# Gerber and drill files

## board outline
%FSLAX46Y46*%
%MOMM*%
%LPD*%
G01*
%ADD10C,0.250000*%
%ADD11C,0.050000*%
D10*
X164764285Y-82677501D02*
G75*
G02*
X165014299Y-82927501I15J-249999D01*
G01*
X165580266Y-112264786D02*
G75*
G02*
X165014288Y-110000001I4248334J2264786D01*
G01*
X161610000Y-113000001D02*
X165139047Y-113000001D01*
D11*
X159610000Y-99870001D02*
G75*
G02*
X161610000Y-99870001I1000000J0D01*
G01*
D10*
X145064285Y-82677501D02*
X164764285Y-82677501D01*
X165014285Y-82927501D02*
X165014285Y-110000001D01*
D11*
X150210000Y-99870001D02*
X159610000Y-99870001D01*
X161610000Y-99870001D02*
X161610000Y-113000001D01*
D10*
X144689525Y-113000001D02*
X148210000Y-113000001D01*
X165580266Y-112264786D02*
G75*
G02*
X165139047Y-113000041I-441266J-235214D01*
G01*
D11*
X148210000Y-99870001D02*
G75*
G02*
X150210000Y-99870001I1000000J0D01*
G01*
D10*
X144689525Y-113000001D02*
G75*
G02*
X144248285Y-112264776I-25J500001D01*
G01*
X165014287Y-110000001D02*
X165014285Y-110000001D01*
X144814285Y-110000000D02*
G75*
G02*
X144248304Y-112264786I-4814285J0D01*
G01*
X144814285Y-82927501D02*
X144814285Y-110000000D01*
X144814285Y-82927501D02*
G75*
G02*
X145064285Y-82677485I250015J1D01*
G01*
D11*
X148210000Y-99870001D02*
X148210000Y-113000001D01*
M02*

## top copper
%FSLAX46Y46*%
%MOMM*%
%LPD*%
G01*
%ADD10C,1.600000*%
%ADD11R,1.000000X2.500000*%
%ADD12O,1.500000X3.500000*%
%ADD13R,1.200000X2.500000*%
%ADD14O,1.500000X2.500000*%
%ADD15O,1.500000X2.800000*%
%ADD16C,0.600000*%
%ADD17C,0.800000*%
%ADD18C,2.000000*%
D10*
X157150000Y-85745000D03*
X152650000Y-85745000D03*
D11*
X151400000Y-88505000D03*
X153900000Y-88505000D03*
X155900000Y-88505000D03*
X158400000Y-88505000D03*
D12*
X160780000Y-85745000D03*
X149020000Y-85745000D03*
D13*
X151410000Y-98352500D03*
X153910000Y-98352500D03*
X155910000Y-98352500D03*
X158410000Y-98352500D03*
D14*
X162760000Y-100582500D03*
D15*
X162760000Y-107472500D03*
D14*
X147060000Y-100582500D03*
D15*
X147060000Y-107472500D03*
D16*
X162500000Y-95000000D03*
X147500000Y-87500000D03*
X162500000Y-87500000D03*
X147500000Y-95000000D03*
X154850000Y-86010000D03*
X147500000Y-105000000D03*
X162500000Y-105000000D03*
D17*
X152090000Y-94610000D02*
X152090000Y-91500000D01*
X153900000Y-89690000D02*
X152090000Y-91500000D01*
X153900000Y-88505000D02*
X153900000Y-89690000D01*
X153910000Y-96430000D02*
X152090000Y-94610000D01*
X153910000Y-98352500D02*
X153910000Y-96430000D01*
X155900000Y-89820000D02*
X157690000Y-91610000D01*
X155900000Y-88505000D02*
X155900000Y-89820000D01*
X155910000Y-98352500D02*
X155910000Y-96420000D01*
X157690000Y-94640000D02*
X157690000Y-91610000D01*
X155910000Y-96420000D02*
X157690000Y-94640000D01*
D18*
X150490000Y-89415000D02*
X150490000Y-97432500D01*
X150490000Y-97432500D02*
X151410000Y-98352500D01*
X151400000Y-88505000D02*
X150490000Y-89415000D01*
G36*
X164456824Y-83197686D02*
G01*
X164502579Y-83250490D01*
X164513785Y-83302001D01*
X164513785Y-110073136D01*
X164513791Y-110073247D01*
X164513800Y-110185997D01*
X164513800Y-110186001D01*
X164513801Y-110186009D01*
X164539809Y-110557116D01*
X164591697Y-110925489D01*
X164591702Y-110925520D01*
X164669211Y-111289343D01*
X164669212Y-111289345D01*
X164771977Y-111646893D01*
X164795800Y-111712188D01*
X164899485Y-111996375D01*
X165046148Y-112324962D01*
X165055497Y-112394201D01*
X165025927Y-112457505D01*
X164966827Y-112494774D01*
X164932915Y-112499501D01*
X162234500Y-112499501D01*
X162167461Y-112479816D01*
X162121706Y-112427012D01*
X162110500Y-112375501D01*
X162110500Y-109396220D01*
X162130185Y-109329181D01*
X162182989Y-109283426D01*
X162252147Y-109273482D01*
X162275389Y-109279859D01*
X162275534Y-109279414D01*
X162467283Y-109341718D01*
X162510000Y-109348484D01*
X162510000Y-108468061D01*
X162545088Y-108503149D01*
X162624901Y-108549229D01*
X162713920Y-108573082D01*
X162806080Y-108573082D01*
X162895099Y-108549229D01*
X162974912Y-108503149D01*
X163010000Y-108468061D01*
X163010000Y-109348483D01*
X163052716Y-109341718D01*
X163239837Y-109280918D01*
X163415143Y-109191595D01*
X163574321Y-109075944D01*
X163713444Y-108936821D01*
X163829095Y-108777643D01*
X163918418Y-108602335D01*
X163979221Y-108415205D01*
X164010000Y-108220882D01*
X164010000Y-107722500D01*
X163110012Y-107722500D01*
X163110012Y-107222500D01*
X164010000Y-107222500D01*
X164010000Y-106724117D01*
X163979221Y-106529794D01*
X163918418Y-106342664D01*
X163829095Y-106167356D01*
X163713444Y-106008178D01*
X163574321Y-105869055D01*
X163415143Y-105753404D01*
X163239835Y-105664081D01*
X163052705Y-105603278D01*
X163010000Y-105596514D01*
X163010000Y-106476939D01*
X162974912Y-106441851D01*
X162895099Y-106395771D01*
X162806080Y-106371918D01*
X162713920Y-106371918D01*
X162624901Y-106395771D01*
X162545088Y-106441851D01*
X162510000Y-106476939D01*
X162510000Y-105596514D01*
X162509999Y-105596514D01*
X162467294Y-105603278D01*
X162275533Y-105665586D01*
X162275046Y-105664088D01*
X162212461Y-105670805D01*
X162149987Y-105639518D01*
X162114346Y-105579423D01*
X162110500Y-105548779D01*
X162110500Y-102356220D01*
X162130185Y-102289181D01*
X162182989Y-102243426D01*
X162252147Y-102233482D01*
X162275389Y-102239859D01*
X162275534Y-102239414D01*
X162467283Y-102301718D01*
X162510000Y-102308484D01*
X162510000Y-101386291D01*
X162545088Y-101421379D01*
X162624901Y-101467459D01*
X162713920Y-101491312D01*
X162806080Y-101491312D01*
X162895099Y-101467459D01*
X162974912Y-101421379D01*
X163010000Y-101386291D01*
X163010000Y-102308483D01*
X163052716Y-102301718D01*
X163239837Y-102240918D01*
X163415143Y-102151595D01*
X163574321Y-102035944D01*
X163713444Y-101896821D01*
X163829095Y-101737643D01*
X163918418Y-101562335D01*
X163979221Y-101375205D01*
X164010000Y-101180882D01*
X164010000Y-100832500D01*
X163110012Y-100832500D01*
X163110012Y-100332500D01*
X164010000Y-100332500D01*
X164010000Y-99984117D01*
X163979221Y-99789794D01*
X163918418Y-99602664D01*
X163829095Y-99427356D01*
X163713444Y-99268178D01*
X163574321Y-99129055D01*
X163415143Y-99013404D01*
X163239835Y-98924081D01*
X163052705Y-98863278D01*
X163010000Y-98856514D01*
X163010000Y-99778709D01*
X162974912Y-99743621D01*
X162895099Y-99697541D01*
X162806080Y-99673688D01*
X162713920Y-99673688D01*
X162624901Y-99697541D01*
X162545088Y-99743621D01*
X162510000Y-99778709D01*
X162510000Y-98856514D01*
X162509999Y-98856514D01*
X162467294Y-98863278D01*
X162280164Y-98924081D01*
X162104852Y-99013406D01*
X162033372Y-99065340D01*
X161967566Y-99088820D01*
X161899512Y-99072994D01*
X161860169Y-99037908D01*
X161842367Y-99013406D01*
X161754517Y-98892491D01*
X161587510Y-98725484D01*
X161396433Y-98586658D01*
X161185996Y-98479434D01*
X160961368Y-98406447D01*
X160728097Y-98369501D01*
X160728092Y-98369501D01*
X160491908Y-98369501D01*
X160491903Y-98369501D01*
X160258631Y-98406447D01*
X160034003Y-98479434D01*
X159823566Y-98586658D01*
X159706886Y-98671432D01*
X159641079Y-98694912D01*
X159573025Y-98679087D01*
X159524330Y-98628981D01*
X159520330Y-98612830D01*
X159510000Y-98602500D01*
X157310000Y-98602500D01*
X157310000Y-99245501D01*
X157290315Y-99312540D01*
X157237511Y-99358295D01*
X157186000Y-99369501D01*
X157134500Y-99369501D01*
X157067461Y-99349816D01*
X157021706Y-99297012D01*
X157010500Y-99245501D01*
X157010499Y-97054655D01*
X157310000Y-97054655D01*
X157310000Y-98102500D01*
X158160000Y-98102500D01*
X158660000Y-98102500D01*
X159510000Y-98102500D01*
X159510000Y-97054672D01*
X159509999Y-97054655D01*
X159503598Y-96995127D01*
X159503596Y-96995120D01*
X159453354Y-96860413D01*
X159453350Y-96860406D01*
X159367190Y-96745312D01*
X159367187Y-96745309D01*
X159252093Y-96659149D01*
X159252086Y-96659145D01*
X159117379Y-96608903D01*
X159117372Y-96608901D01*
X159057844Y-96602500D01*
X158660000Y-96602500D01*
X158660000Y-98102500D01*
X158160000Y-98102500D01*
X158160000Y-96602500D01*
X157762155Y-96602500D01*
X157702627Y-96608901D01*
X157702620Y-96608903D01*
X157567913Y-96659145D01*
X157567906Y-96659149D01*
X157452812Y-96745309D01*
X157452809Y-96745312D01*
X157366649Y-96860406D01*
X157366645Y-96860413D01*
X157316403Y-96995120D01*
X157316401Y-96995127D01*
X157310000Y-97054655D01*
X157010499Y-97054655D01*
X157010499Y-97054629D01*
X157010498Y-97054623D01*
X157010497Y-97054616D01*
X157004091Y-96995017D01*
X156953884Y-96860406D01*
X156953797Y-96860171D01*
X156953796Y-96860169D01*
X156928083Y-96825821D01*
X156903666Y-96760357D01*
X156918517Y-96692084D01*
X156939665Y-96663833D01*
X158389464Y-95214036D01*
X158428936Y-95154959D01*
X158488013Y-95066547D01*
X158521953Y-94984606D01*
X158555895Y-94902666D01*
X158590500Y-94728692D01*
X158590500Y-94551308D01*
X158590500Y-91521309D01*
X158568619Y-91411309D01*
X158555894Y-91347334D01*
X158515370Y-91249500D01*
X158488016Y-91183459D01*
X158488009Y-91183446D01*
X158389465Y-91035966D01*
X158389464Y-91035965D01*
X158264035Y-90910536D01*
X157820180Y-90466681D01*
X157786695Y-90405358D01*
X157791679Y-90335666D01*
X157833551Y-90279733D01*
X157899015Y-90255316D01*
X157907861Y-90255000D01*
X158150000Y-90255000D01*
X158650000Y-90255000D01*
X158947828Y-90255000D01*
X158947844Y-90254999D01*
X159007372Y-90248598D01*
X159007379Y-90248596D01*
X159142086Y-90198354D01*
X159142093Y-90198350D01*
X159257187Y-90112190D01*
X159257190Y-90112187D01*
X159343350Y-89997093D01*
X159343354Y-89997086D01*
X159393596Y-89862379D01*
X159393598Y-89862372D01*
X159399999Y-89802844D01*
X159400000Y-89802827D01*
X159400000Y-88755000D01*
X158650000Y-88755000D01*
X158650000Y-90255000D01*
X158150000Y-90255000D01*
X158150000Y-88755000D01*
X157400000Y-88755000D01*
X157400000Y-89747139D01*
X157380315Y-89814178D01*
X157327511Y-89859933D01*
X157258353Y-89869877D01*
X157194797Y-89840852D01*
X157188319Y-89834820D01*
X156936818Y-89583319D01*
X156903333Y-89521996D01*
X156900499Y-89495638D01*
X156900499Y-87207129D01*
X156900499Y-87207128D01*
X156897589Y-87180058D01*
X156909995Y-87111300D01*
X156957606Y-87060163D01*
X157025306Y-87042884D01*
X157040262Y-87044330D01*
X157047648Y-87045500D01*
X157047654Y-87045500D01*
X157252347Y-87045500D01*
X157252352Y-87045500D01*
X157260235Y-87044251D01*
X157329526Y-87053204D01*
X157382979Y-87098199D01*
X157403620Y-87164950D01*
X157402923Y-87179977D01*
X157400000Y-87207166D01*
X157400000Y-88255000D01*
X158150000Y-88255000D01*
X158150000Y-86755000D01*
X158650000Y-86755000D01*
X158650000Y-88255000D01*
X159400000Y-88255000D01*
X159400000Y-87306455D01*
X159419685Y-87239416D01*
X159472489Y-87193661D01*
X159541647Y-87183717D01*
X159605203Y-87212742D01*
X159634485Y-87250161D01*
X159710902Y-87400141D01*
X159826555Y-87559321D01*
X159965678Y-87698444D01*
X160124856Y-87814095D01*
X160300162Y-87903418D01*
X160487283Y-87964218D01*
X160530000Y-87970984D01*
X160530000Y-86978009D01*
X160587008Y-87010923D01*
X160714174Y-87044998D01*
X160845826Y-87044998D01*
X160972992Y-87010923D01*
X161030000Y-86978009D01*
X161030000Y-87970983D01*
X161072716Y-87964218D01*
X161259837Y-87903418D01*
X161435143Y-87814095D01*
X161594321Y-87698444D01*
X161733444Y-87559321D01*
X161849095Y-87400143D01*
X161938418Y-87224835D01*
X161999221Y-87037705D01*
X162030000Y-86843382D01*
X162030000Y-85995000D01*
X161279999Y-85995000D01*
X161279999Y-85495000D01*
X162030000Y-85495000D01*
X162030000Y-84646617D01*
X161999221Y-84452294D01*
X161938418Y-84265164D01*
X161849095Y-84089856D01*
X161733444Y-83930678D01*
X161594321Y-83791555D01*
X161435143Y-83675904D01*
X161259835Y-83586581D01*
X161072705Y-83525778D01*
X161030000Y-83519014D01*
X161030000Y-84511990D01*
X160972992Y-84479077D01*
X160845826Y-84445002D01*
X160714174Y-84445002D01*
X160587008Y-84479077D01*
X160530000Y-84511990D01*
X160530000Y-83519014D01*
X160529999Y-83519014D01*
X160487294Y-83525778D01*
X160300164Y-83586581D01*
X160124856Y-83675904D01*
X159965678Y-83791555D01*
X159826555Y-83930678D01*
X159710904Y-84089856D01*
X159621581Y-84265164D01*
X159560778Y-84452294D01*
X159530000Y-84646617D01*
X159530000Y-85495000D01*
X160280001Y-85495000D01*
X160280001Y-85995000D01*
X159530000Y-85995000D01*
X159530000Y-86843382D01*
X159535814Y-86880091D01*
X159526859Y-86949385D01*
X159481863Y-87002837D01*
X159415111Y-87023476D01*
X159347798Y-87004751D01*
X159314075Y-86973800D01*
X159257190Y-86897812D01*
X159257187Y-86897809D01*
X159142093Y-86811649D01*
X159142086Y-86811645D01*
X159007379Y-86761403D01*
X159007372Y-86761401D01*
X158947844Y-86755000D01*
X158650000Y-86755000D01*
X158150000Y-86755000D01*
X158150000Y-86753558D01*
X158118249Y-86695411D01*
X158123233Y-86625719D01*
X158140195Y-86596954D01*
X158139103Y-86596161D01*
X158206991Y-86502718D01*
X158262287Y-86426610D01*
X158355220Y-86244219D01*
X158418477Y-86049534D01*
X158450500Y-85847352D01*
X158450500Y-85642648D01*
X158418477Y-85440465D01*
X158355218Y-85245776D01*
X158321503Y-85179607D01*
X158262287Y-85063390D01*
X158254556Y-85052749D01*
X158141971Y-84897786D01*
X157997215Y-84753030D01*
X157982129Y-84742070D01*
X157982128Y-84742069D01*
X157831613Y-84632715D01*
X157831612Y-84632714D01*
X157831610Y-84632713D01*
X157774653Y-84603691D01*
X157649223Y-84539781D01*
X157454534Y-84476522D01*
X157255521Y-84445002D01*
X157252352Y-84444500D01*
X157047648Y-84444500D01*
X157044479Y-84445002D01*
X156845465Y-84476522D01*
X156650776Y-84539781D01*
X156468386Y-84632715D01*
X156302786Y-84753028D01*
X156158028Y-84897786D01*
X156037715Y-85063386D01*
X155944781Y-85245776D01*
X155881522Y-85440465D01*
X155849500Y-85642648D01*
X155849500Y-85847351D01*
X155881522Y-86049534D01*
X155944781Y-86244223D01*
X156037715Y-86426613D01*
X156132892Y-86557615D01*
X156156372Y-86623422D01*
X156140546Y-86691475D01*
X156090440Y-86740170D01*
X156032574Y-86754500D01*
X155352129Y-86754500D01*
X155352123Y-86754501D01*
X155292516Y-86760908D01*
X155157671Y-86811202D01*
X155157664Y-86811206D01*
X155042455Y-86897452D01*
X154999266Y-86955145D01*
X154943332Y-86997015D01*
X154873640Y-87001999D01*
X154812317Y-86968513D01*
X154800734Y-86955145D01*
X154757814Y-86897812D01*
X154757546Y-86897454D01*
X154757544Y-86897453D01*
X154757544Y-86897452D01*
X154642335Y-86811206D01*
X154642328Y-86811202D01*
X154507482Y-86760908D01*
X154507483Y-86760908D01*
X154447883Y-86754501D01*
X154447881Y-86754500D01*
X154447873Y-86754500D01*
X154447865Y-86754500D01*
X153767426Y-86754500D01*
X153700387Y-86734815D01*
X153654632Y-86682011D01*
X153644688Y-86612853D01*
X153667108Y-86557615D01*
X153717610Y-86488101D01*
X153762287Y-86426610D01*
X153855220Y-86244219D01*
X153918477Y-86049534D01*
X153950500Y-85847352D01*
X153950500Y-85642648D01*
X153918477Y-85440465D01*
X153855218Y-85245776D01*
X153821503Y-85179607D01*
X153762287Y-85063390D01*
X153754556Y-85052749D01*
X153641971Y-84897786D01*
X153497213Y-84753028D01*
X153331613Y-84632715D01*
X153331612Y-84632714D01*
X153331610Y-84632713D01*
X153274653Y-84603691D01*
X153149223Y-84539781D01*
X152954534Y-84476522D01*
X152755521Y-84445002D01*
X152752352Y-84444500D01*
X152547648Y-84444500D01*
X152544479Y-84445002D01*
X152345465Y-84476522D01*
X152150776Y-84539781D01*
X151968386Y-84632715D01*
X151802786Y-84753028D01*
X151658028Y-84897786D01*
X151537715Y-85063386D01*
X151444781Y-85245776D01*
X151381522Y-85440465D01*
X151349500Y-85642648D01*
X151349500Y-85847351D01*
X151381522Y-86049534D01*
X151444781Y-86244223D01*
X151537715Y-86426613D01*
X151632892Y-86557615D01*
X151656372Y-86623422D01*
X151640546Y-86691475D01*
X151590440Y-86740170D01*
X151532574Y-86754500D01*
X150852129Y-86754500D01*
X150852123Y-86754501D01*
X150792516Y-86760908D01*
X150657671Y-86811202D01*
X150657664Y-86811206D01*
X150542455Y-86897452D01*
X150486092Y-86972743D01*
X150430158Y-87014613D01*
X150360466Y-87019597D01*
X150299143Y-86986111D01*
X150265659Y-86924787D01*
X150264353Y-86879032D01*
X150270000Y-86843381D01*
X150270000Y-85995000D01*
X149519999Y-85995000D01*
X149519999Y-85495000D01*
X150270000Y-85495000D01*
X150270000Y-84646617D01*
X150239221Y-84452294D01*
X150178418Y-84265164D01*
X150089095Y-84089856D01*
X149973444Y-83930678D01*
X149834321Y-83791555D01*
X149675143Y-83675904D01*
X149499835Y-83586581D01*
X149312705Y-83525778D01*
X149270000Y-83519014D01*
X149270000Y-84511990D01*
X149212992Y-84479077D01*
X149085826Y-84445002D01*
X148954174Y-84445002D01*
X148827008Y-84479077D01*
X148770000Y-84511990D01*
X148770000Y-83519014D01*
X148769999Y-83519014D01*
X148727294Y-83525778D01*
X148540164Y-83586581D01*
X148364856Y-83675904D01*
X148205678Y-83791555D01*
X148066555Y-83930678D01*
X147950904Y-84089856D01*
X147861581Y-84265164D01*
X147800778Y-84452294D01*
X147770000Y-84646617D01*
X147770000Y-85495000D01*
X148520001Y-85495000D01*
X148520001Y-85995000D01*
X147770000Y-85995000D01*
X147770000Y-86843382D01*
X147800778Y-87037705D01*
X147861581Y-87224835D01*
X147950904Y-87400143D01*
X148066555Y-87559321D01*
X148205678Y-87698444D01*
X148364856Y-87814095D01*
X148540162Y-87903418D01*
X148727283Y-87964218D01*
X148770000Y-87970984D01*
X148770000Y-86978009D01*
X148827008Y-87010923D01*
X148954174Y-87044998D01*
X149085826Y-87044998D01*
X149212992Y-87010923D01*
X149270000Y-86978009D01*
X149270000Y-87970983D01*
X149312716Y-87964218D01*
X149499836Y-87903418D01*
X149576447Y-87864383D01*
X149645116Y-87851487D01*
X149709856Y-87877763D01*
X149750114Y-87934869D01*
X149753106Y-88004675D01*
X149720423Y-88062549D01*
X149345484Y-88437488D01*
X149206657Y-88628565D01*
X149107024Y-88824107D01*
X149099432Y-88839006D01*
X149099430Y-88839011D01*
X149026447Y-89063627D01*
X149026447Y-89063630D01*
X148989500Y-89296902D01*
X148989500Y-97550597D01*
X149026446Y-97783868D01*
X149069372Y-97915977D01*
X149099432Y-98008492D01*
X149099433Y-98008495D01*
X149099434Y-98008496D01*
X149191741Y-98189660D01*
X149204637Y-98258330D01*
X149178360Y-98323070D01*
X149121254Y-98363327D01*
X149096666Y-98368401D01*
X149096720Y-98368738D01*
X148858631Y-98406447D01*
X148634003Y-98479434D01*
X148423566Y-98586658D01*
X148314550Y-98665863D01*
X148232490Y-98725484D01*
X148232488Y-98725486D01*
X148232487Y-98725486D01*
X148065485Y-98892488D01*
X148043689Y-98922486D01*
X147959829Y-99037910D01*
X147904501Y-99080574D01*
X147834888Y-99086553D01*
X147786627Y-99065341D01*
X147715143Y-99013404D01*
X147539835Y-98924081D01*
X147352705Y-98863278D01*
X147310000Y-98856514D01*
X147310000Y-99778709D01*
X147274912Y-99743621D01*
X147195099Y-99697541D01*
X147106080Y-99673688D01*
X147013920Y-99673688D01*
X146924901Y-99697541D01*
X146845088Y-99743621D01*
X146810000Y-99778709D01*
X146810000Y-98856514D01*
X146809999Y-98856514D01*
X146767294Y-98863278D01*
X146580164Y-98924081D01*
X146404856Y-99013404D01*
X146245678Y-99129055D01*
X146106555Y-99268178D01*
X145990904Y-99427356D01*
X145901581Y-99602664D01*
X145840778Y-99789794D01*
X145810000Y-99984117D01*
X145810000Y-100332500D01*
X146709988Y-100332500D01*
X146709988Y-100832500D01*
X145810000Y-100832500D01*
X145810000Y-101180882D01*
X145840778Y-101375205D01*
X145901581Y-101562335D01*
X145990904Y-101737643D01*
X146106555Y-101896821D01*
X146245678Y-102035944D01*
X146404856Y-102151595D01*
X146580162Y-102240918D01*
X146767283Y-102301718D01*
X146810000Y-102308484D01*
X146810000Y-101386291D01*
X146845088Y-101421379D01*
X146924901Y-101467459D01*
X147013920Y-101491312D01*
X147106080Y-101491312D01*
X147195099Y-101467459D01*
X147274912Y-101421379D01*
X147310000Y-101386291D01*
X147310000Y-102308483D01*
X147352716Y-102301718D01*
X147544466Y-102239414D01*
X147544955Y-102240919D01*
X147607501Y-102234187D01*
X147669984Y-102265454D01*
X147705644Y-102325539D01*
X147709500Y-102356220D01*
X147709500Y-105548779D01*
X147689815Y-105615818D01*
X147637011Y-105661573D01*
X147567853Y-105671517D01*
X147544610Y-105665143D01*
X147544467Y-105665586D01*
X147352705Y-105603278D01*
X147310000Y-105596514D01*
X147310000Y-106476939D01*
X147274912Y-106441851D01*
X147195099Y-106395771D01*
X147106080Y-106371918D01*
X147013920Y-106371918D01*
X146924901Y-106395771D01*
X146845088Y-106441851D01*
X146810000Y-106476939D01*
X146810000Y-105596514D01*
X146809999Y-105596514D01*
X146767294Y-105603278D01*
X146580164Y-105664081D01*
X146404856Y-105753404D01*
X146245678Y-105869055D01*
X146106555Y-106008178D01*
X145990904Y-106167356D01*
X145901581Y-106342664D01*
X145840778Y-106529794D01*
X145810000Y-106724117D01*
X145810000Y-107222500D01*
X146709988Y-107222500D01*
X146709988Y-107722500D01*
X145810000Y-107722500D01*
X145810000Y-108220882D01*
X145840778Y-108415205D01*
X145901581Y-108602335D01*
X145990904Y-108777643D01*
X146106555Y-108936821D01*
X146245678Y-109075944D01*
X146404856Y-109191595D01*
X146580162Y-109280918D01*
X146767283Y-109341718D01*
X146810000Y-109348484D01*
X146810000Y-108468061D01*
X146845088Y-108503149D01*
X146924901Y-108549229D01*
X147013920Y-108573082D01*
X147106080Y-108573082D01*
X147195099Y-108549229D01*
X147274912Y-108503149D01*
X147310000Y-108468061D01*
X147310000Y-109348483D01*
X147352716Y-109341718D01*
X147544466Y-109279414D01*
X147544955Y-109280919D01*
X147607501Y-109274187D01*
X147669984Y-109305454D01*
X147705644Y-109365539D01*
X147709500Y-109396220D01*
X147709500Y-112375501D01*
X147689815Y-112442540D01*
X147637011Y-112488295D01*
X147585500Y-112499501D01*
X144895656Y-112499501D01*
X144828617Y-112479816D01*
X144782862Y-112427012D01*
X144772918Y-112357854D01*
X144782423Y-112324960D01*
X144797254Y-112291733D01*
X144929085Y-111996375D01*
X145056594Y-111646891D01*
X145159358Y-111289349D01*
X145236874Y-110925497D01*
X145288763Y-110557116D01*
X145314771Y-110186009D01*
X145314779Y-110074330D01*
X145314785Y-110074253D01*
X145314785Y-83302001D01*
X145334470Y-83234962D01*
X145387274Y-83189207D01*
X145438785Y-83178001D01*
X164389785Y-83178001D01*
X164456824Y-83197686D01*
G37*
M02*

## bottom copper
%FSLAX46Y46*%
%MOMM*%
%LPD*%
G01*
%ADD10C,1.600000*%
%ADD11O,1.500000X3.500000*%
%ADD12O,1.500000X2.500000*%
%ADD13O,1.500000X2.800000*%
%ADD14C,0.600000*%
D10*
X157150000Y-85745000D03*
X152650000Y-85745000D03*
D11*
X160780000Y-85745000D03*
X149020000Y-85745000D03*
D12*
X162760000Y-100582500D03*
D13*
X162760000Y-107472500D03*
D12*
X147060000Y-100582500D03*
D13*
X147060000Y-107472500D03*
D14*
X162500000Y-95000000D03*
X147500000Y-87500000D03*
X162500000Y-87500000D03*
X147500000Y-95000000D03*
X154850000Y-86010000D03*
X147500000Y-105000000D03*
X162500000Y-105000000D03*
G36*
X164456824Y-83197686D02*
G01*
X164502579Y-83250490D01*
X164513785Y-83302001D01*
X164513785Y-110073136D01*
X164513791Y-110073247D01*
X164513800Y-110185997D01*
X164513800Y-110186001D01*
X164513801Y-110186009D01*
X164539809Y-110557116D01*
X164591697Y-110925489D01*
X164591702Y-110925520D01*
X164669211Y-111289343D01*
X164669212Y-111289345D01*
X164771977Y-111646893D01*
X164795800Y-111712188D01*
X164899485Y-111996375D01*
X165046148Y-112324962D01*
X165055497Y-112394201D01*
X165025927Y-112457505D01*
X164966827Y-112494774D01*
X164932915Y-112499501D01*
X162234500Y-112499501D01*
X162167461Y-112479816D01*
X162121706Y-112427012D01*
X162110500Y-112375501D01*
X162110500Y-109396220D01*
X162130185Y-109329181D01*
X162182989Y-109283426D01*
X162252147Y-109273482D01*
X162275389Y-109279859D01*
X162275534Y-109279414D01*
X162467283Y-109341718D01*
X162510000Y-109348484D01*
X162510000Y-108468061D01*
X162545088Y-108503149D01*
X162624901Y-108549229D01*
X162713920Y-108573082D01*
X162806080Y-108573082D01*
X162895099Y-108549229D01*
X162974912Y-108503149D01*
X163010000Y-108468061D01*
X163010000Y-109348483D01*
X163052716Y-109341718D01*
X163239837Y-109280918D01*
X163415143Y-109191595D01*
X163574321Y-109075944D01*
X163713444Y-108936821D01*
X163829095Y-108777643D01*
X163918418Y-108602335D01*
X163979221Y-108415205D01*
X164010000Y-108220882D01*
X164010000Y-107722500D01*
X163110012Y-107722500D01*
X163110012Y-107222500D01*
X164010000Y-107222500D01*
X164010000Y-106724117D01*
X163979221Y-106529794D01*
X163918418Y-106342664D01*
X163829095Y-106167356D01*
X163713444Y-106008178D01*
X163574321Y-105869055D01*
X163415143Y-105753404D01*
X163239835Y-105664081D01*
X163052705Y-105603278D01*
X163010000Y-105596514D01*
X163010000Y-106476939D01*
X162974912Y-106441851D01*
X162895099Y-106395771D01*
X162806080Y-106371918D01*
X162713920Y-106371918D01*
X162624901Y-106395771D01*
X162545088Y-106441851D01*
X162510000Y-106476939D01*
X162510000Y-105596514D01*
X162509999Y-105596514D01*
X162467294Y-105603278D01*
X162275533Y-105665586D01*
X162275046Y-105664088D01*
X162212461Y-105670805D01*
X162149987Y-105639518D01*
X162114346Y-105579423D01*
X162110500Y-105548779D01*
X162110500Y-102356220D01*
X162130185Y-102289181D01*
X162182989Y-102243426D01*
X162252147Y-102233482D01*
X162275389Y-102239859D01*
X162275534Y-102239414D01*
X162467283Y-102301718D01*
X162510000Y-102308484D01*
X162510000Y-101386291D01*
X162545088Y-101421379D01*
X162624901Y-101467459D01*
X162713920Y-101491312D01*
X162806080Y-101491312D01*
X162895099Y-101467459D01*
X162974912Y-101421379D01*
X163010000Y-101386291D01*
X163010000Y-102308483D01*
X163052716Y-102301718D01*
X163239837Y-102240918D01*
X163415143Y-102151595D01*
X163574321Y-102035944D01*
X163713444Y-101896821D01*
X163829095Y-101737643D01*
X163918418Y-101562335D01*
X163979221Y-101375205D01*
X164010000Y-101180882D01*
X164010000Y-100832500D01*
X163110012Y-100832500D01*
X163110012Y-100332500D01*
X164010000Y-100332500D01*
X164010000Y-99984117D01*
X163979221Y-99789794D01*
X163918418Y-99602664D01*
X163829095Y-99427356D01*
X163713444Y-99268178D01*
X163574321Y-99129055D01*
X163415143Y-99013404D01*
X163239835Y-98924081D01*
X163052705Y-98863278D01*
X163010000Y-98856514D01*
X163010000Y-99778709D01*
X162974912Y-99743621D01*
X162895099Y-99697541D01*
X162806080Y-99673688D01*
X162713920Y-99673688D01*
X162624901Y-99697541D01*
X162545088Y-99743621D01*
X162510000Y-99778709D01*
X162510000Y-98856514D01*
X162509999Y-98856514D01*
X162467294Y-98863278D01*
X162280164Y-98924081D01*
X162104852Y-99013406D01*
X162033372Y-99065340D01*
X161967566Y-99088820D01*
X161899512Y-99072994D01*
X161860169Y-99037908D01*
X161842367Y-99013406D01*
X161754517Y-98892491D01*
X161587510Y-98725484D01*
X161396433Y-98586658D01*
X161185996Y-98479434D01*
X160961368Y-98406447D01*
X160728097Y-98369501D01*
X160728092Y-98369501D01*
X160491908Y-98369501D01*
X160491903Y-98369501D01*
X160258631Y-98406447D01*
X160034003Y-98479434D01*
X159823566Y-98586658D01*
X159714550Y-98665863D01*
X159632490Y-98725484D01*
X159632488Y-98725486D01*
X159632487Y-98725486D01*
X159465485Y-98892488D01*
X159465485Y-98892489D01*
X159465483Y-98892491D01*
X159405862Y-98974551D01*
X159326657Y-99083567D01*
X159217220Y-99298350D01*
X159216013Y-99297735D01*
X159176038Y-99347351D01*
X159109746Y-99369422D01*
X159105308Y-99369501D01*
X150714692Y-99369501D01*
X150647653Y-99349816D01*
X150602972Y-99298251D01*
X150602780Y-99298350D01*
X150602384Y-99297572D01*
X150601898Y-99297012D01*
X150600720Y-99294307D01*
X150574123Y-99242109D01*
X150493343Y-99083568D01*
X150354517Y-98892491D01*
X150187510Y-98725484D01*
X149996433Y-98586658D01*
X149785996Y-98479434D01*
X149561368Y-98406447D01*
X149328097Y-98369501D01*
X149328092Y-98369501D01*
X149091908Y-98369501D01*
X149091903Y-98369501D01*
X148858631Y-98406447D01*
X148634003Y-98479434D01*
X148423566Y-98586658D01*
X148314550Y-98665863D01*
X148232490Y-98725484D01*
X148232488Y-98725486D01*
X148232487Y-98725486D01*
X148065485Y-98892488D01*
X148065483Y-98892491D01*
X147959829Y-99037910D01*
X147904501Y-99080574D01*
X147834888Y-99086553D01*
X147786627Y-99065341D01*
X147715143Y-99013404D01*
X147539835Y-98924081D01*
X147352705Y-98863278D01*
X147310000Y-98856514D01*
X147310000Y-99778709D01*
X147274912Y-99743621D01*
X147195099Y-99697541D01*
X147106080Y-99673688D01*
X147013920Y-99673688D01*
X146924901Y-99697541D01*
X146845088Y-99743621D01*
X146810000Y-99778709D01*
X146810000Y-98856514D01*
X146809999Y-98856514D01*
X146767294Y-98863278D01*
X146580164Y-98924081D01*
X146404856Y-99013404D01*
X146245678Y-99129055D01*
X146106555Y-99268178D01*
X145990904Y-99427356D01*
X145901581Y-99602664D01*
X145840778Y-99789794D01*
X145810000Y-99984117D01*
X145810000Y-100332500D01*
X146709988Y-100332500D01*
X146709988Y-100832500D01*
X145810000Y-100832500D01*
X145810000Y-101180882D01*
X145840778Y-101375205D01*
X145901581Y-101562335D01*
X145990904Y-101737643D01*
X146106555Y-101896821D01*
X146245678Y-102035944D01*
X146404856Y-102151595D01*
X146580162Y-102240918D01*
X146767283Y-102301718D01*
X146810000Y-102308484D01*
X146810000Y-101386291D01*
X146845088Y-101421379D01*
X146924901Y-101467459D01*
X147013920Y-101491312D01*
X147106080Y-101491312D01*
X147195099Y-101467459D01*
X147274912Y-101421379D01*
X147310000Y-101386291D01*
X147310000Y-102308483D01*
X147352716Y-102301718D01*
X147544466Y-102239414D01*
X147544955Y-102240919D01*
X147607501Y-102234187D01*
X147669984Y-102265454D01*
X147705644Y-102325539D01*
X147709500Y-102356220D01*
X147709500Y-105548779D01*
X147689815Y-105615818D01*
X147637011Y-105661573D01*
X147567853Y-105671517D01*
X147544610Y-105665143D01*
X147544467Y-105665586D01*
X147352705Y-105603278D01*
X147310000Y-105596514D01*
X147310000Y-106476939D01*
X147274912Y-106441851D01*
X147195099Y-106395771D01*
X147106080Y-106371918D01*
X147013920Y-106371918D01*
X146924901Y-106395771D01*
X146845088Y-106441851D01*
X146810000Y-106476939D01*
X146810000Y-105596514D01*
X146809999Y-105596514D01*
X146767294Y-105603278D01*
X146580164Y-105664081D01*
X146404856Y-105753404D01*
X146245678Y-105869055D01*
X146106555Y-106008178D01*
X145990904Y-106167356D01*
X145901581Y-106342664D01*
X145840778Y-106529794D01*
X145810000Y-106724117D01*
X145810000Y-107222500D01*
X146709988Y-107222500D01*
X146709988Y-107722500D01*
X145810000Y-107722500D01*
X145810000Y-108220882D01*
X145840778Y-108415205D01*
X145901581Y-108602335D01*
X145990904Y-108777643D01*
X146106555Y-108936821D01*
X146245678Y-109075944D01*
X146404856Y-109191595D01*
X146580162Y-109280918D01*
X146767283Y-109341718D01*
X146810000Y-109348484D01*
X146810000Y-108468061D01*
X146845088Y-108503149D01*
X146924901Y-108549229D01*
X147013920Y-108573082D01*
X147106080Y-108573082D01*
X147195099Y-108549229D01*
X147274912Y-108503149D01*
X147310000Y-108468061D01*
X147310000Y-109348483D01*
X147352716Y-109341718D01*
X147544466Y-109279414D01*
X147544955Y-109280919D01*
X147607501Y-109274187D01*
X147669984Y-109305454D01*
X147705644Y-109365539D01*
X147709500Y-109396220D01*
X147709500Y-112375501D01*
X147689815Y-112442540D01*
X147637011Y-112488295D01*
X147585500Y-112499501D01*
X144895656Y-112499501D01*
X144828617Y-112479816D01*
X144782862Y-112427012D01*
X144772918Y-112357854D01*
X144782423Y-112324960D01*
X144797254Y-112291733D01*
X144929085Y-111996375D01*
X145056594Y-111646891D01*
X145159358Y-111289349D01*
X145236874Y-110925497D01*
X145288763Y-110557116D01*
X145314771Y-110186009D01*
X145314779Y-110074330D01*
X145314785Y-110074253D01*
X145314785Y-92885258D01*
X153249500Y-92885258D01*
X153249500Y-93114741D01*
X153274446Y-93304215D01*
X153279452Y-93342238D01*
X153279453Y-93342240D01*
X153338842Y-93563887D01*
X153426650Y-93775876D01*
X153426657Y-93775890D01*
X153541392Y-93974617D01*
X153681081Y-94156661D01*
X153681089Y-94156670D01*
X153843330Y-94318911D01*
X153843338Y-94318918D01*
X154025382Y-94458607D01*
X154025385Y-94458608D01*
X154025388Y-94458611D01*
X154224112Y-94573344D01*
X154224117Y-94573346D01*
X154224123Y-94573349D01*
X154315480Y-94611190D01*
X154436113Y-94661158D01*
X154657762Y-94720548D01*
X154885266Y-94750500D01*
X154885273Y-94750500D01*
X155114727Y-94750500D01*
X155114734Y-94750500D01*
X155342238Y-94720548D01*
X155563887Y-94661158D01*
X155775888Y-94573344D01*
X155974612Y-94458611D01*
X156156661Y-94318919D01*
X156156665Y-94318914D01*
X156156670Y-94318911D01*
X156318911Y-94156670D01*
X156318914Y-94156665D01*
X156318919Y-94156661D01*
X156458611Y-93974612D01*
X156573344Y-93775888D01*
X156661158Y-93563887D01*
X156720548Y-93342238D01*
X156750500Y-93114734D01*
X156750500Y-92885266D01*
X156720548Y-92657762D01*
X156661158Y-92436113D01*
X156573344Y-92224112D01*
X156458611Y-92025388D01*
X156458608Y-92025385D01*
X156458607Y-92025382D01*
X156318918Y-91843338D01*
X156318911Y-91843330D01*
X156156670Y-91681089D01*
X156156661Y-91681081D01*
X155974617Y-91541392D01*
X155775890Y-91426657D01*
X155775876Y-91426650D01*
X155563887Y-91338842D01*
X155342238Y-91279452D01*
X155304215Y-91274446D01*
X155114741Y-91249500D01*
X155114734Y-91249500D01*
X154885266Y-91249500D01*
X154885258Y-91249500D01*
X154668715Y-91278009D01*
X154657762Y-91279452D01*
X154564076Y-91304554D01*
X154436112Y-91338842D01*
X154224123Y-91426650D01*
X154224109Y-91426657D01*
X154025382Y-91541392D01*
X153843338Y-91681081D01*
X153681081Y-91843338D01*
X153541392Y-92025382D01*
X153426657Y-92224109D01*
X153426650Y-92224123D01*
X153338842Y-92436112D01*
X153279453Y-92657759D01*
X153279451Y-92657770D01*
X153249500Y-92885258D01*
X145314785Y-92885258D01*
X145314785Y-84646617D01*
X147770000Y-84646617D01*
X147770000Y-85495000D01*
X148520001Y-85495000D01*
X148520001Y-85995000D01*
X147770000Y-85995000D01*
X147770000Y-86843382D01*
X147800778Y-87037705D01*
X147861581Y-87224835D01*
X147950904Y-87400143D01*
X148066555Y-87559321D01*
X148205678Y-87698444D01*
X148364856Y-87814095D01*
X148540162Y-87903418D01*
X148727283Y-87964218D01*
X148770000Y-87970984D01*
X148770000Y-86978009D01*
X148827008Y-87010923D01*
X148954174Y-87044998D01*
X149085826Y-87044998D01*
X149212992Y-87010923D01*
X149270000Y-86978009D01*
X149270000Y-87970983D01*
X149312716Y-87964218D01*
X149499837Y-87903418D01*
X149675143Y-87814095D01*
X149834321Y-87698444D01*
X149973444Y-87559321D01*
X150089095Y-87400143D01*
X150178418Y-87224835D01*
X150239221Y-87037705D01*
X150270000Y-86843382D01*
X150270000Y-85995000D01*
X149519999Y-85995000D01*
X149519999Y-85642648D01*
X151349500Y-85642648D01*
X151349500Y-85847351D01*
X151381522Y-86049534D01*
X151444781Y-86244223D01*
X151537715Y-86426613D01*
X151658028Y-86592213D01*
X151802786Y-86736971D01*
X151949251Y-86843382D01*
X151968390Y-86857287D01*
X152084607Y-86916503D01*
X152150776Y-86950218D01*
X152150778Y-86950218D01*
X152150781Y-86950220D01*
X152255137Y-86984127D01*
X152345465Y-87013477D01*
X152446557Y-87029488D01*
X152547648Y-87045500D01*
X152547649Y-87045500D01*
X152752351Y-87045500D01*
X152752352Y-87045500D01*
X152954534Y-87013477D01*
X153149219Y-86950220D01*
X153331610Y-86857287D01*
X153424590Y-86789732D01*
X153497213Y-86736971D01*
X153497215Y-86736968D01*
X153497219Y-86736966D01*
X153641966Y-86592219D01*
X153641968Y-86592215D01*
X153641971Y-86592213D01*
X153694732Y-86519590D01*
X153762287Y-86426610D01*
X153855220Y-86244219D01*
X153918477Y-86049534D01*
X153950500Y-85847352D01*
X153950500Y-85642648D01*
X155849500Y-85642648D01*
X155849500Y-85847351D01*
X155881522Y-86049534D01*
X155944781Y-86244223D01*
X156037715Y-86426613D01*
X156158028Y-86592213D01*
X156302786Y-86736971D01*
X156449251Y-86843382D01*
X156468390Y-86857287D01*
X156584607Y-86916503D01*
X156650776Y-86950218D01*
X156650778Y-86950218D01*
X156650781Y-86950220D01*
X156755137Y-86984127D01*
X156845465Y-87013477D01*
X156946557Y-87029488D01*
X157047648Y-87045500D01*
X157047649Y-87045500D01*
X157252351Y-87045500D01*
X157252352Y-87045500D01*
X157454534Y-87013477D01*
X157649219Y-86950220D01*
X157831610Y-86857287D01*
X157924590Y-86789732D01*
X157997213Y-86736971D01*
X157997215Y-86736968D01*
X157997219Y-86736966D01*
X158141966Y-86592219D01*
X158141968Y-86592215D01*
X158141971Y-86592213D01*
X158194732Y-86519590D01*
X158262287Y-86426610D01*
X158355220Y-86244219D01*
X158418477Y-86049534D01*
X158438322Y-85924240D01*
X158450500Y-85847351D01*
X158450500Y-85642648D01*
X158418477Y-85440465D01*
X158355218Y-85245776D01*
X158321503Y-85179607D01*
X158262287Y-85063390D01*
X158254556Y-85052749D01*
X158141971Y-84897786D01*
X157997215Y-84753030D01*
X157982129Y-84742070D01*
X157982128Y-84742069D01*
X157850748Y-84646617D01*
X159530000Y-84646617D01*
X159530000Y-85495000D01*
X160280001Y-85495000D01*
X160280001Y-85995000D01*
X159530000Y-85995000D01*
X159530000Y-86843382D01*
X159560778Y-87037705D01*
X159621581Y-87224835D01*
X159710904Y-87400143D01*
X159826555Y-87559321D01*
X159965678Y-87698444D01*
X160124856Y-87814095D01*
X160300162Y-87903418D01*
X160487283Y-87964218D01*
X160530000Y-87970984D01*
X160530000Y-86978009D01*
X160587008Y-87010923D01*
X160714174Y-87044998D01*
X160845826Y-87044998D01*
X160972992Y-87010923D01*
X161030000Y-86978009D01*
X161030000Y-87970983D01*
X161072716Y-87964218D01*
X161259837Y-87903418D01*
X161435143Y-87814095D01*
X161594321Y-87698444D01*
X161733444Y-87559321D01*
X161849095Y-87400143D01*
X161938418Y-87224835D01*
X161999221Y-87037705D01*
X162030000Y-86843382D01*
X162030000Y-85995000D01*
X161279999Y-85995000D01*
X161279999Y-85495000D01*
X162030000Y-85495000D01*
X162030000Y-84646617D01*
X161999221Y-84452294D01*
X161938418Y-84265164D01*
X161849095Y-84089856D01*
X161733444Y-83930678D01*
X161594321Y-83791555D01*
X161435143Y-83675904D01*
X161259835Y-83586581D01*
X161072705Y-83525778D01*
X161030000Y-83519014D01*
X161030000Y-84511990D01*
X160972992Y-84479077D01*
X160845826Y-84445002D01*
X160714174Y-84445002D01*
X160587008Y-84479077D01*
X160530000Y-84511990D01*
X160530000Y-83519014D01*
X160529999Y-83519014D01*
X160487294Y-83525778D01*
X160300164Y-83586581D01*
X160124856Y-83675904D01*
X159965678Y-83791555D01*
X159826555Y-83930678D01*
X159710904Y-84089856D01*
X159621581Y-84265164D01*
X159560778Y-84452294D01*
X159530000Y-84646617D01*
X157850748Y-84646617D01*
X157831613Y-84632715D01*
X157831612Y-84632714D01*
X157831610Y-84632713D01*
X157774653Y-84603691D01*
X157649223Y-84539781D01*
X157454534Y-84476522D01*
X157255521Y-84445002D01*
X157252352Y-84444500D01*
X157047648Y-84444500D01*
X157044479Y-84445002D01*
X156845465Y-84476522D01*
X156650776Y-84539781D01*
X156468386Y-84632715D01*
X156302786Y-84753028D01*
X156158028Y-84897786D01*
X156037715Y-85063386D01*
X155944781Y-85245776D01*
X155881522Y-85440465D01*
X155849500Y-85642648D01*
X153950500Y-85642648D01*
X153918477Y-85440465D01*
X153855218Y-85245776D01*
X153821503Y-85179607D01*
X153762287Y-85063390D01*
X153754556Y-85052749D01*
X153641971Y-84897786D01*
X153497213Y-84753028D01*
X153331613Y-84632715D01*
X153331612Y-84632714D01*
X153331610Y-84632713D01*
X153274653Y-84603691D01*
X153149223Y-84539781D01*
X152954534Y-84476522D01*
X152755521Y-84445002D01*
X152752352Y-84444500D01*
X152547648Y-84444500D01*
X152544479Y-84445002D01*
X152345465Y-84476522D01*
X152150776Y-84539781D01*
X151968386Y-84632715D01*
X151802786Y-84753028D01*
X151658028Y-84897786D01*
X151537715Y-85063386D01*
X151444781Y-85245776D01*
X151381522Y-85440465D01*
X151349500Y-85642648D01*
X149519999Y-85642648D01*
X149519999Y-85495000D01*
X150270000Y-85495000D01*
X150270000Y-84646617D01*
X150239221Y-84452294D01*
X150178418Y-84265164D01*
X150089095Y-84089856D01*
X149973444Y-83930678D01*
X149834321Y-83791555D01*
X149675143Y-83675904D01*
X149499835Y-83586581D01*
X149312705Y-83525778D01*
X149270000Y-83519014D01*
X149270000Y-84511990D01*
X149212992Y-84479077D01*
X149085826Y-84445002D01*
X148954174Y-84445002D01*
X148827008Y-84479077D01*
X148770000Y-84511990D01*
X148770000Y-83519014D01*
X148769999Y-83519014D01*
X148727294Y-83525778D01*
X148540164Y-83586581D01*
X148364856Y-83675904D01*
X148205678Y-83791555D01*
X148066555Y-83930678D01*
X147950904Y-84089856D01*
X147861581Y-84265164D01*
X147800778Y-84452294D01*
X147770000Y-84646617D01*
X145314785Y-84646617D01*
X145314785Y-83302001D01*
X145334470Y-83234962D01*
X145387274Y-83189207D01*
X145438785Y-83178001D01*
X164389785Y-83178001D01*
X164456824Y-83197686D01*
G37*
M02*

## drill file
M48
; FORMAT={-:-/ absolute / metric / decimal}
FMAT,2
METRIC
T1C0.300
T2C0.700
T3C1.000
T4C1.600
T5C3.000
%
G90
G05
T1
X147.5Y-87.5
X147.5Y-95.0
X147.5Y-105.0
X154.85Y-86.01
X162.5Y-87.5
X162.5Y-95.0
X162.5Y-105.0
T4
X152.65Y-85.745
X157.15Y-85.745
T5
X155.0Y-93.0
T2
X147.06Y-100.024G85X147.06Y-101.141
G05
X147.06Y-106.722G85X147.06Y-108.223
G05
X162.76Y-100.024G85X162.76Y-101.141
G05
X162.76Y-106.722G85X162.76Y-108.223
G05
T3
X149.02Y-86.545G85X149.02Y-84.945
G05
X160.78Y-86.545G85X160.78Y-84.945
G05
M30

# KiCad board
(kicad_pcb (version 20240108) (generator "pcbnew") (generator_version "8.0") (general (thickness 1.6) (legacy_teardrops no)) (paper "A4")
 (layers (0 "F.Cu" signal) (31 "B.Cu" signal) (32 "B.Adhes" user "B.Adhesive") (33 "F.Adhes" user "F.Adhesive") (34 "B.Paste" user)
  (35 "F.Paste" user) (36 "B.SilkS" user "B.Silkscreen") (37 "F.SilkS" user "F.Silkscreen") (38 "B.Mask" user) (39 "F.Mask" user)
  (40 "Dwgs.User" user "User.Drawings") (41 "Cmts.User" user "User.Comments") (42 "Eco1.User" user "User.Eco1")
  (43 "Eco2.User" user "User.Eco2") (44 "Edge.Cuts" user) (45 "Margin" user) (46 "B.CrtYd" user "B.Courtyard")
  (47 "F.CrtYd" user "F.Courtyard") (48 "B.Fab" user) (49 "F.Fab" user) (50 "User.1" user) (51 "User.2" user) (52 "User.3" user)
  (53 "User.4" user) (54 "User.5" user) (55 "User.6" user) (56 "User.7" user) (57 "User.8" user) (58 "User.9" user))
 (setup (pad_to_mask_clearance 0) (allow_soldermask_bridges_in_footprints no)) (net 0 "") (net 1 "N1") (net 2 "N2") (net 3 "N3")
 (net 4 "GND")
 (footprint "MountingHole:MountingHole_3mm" (layer "F.Cu") (at 155 93)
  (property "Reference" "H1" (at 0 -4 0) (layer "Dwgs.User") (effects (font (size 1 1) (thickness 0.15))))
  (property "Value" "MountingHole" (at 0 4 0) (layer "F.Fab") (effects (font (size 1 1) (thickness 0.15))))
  (pad "" np_thru_hole circle (at 0 0) (size 3 3) (drill 3) (layers "*.Cu" "*.Mask")))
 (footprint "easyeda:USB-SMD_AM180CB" (layer "F.Cu") (at 154.9 87.125 180)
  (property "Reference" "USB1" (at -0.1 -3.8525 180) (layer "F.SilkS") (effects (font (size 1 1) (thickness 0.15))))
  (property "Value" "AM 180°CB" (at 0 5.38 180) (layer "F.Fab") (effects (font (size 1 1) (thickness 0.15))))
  (pad "" thru_hole circle (at -2.25 1.38 180) (size 1.6 1.6) (drill 1.6) (layers "*.Cu" "*.Mask") (remove_unused_layers no))
  (pad "" thru_hole circle (at 2.25 1.38 180) (size 1.6 1.6) (drill 1.6) (layers "*.Cu" "*.Mask") (remove_unused_layers no))
  (pad "1" smd rect (at 3.5 -1.38 180) (size 1 2.5) (layers "F.Cu" "F.Paste" "F.Mask") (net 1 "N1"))
  (pad "2" smd rect (at 1 -1.38 180) (size 1 2.5) (layers "F.Cu" "F.Paste" "F.Mask") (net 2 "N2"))
  (pad "3" smd rect (at -1 -1.38 180) (size 1 2.5) (layers "F.Cu" "F.Paste" "F.Mask") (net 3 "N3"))
  (pad "4" smd rect (at -3.5 -1.38 180) (size 1 2.5) (layers "F.Cu" "F.Paste" "F.Mask") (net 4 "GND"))
  (pad "5" thru_hole oval (at -5.88 1.38 180) (size 1.5 3.5) (drill oval 0.999998 2.599995) (layers "*.Cu" "*.Mask")
   (remove_unused_layers no) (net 4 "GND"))
  (pad "5" thru_hole oval (at 5.88 1.38 180) (size 1.5 3.5) (drill oval 0.999998 2.599995) (layers "*.Cu" "*.Mask")
   (remove_unused_layers no) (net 4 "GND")))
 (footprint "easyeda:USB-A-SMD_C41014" (layer "F.Cu") (at 154.91 102.9125)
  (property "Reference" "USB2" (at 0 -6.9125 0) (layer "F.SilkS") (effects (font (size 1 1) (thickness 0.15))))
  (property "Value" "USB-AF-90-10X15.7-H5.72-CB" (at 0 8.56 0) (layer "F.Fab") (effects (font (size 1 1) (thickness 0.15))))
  (pad "1" smd rect (at -3.5 -4.56) (size 1.2 2.5) (layers "F.Cu" "F.Paste" "F.Mask") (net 1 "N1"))
  (pad "2" smd rect (at -1 -4.56) (size 1.2 2.5) (layers "F.Cu" "F.Paste" "F.Mask") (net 2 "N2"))
  (pad "3" smd rect (at 1 -4.56) (size 1.2 2.5) (layers "F.Cu" "F.Paste" "F.Mask") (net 3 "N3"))
  (pad "4" smd rect (at 3.5 -4.56) (size 1.2 2.5) (layers "F.Cu" "F.Paste" "F.Mask") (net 4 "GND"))
  (pad "5" thru_hole oval (at 7.85 -2.33) (size 1.5 2.5) (drill oval 0.700024 1.817624) (layers "*.Cu" "*.Mask") (remove_unused_layers no)
   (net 4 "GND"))
  (pad "6" thru_hole oval (at 7.85 4.56) (size 1.5 2.8) (drill oval 0.700024 2.201164) (layers "*.Cu" "*.Mask") (remove_unused_layers no)
   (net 4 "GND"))
  (pad "7" thru_hole oval (at -7.85 -2.33) (size 1.5 2.5) (drill oval 0.700024 1.817624) (layers "*.Cu" "*.Mask") (remove_unused_layers no)
   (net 4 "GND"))
  (pad "8" thru_hole oval (at -7.85 4.56) (size 1.5 2.8) (drill oval 0.700024 2.201164) (layers "*.Cu" "*.Mask") (remove_unused_layers no)
   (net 4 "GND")))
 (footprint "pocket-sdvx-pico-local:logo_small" (layer "B.Cu") (at 149 93 180)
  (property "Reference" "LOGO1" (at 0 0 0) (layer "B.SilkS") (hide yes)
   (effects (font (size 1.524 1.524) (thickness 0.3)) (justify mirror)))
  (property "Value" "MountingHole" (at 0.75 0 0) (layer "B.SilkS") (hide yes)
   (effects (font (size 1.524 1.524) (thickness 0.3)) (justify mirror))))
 (gr_arc (start 164.764285 82.677501) (mid 164.941063 82.750722) (end 165.014285 82.927501) (stroke (width 0.25) (type default))
  (layer "Edge.Cuts"))
 (gr_arc (start 165.580266 112.264786) (mid 165.157924 111.167218) (end 165.014287 110.000001) (stroke (width 0.25) (type default))
  (layer "Edge.Cuts"))
 (gr_line (start 161.61 113.000001) (end 165.139047 113.000001) (stroke (width 0.25) (type default)) (layer "Edge.Cuts"))
 (gr_arc (start 159.61 99.870001) (mid 160.61 98.870001) (end 161.61 99.870001) (stroke (width 0.05) (type default)) (layer "Edge.Cuts"))
 (gr_line (start 145.064285 82.677501) (end 164.764285 82.677501) (stroke (width 0.25) (type default)) (layer "Edge.Cuts"))
 (gr_line (start 165.014285 82.927501) (end 165.014285 110.000001) (stroke (width 0.25) (type default)) (layer "Edge.Cuts"))
 (gr_line (start 150.21 99.870001) (end 159.61 99.870001) (stroke (width 0.05) (type default)) (layer "Edge.Cuts"))
 (gr_line (start 161.61 99.870001) (end 161.61 113.000001) (stroke (width 0.05) (type default)) (layer "Edge.Cuts"))
 (gr_line (start 144.689525 113.000001) (end 148.21 113.000001) (stroke (width 0.25) (type default)) (layer "Edge.Cuts"))
 (gr_arc (start 165.580266 112.264786) (mid 165.567775 112.757279) (end 165.139047 113.000001) (stroke (width 0.25) (type default))
  (layer "Edge.Cuts"))
 (gr_arc (start 148.21 99.870001) (mid 149.21 98.870001) (end 150.21 99.870001) (stroke (width 0.05) (type default)) (layer "Edge.Cuts"))
 (gr_arc (start 144.689525 113.000001) (mid 144.2608 112.757288) (end 144.248304 112.264786) (stroke (width 0.25) (type default))
  (layer "Edge.Cuts"))
 (gr_line (start 165.014287 110.000001) (end 165.014285 110.000001) (stroke (width 0.25) (type default)) (layer "Edge.Cuts"))
 (gr_arc (start 144.814285 110) (mid 144.670647 111.167218) (end 144.248304 112.264786) (stroke (width 0.25) (type default))
  (layer "Edge.Cuts"))
 (gr_line (start 144.814285 82.927501) (end 144.814285 110) (stroke (width 0.25) (type default)) (layer "Edge.Cuts"))
 (gr_arc (start 144.814285 82.927501) (mid 144.88751 82.750726) (end 145.064285 82.677501) (stroke (width 0.25) (type default))
  (layer "Edge.Cuts"))
 (gr_line (start 148.21 99.870001) (end 148.21 113.000001) (stroke (width 0.05) (type default)) (layer "Edge.Cuts"))
 (segment (start 152.09 94.61) (end 152.09 91.5) (width 0.8) (layer "F.Cu") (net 2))
 (segment (start 153.9 89.69) (end 152.09 91.5) (width 0.8) (layer "F.Cu") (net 2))
 (segment (start 153.9 88.505) (end 153.9 89.69) (width 0.8) (layer "F.Cu") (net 2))
 (segment (start 153.91 96.43) (end 152.09 94.61) (width 0.8) (layer "F.Cu") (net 2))
 (segment (start 153.91 98.3525) (end 153.91 96.43) (width 0.8) (layer "F.Cu") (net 2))
 (segment (start 155.9 89.82) (end 157.69 91.61) (width 0.8) (layer "F.Cu") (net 3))
 (segment (start 155.9 88.505) (end 155.9 89.82) (width 0.8) (layer "F.Cu") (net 3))
 (segment (start 155.91 98.3525) (end 155.91 96.42) (width 0.8) (layer "F.Cu") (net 3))
 (segment (start 157.69 94.64) (end 157.69 91.61) (width 0.8) (layer "F.Cu") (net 3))
 (segment (start 155.91 96.42) (end 157.69 94.64) (width 0.8) (layer "F.Cu") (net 3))
 (segment (start 150.49 89.415) (end 150.49 97.4325) (width 2) (layer "F.Cu") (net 1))
 (segment (start 150.49 97.4325) (end 151.41 98.3525) (width 2) (layer "F.Cu") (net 1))
 (segment (start 151.4 88.505) (end 150.49 89.415) (width 2) (layer "F.Cu") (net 1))
 (via (at 162.5 95) (size 0.6) (drill 0.3) (layers "F.Cu" "B.Cu") (free yes) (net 4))
 (via (at 147.5 87.5) (size 0.6) (drill 0.3) (layers "F.Cu" "B.Cu") (free yes) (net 4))
 (via (at 162.5 87.5) (size 0.6) (drill 0.3) (layers "F.Cu" "B.Cu") (free yes) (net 4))
 (via (at 147.5 95) (size 0.6) (drill 0.3) (layers "F.Cu" "B.Cu") (free yes) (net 4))
 (via (at 154.85 86.01) (size 0.6) (drill 0.3) (layers "F.Cu" "B.Cu") (free yes) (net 4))
 (via (at 147.5 105) (size 0.6) (drill 0.3) (layers "F.Cu" "B.Cu") (free yes) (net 4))
 (via (at 162.5 105) (size 0.6) (drill 0.3) (layers "F.Cu" "B.Cu") (free yes) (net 4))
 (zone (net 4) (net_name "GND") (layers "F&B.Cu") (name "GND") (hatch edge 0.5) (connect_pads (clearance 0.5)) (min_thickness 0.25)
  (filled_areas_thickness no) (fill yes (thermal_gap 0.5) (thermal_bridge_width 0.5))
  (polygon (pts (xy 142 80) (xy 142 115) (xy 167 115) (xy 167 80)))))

